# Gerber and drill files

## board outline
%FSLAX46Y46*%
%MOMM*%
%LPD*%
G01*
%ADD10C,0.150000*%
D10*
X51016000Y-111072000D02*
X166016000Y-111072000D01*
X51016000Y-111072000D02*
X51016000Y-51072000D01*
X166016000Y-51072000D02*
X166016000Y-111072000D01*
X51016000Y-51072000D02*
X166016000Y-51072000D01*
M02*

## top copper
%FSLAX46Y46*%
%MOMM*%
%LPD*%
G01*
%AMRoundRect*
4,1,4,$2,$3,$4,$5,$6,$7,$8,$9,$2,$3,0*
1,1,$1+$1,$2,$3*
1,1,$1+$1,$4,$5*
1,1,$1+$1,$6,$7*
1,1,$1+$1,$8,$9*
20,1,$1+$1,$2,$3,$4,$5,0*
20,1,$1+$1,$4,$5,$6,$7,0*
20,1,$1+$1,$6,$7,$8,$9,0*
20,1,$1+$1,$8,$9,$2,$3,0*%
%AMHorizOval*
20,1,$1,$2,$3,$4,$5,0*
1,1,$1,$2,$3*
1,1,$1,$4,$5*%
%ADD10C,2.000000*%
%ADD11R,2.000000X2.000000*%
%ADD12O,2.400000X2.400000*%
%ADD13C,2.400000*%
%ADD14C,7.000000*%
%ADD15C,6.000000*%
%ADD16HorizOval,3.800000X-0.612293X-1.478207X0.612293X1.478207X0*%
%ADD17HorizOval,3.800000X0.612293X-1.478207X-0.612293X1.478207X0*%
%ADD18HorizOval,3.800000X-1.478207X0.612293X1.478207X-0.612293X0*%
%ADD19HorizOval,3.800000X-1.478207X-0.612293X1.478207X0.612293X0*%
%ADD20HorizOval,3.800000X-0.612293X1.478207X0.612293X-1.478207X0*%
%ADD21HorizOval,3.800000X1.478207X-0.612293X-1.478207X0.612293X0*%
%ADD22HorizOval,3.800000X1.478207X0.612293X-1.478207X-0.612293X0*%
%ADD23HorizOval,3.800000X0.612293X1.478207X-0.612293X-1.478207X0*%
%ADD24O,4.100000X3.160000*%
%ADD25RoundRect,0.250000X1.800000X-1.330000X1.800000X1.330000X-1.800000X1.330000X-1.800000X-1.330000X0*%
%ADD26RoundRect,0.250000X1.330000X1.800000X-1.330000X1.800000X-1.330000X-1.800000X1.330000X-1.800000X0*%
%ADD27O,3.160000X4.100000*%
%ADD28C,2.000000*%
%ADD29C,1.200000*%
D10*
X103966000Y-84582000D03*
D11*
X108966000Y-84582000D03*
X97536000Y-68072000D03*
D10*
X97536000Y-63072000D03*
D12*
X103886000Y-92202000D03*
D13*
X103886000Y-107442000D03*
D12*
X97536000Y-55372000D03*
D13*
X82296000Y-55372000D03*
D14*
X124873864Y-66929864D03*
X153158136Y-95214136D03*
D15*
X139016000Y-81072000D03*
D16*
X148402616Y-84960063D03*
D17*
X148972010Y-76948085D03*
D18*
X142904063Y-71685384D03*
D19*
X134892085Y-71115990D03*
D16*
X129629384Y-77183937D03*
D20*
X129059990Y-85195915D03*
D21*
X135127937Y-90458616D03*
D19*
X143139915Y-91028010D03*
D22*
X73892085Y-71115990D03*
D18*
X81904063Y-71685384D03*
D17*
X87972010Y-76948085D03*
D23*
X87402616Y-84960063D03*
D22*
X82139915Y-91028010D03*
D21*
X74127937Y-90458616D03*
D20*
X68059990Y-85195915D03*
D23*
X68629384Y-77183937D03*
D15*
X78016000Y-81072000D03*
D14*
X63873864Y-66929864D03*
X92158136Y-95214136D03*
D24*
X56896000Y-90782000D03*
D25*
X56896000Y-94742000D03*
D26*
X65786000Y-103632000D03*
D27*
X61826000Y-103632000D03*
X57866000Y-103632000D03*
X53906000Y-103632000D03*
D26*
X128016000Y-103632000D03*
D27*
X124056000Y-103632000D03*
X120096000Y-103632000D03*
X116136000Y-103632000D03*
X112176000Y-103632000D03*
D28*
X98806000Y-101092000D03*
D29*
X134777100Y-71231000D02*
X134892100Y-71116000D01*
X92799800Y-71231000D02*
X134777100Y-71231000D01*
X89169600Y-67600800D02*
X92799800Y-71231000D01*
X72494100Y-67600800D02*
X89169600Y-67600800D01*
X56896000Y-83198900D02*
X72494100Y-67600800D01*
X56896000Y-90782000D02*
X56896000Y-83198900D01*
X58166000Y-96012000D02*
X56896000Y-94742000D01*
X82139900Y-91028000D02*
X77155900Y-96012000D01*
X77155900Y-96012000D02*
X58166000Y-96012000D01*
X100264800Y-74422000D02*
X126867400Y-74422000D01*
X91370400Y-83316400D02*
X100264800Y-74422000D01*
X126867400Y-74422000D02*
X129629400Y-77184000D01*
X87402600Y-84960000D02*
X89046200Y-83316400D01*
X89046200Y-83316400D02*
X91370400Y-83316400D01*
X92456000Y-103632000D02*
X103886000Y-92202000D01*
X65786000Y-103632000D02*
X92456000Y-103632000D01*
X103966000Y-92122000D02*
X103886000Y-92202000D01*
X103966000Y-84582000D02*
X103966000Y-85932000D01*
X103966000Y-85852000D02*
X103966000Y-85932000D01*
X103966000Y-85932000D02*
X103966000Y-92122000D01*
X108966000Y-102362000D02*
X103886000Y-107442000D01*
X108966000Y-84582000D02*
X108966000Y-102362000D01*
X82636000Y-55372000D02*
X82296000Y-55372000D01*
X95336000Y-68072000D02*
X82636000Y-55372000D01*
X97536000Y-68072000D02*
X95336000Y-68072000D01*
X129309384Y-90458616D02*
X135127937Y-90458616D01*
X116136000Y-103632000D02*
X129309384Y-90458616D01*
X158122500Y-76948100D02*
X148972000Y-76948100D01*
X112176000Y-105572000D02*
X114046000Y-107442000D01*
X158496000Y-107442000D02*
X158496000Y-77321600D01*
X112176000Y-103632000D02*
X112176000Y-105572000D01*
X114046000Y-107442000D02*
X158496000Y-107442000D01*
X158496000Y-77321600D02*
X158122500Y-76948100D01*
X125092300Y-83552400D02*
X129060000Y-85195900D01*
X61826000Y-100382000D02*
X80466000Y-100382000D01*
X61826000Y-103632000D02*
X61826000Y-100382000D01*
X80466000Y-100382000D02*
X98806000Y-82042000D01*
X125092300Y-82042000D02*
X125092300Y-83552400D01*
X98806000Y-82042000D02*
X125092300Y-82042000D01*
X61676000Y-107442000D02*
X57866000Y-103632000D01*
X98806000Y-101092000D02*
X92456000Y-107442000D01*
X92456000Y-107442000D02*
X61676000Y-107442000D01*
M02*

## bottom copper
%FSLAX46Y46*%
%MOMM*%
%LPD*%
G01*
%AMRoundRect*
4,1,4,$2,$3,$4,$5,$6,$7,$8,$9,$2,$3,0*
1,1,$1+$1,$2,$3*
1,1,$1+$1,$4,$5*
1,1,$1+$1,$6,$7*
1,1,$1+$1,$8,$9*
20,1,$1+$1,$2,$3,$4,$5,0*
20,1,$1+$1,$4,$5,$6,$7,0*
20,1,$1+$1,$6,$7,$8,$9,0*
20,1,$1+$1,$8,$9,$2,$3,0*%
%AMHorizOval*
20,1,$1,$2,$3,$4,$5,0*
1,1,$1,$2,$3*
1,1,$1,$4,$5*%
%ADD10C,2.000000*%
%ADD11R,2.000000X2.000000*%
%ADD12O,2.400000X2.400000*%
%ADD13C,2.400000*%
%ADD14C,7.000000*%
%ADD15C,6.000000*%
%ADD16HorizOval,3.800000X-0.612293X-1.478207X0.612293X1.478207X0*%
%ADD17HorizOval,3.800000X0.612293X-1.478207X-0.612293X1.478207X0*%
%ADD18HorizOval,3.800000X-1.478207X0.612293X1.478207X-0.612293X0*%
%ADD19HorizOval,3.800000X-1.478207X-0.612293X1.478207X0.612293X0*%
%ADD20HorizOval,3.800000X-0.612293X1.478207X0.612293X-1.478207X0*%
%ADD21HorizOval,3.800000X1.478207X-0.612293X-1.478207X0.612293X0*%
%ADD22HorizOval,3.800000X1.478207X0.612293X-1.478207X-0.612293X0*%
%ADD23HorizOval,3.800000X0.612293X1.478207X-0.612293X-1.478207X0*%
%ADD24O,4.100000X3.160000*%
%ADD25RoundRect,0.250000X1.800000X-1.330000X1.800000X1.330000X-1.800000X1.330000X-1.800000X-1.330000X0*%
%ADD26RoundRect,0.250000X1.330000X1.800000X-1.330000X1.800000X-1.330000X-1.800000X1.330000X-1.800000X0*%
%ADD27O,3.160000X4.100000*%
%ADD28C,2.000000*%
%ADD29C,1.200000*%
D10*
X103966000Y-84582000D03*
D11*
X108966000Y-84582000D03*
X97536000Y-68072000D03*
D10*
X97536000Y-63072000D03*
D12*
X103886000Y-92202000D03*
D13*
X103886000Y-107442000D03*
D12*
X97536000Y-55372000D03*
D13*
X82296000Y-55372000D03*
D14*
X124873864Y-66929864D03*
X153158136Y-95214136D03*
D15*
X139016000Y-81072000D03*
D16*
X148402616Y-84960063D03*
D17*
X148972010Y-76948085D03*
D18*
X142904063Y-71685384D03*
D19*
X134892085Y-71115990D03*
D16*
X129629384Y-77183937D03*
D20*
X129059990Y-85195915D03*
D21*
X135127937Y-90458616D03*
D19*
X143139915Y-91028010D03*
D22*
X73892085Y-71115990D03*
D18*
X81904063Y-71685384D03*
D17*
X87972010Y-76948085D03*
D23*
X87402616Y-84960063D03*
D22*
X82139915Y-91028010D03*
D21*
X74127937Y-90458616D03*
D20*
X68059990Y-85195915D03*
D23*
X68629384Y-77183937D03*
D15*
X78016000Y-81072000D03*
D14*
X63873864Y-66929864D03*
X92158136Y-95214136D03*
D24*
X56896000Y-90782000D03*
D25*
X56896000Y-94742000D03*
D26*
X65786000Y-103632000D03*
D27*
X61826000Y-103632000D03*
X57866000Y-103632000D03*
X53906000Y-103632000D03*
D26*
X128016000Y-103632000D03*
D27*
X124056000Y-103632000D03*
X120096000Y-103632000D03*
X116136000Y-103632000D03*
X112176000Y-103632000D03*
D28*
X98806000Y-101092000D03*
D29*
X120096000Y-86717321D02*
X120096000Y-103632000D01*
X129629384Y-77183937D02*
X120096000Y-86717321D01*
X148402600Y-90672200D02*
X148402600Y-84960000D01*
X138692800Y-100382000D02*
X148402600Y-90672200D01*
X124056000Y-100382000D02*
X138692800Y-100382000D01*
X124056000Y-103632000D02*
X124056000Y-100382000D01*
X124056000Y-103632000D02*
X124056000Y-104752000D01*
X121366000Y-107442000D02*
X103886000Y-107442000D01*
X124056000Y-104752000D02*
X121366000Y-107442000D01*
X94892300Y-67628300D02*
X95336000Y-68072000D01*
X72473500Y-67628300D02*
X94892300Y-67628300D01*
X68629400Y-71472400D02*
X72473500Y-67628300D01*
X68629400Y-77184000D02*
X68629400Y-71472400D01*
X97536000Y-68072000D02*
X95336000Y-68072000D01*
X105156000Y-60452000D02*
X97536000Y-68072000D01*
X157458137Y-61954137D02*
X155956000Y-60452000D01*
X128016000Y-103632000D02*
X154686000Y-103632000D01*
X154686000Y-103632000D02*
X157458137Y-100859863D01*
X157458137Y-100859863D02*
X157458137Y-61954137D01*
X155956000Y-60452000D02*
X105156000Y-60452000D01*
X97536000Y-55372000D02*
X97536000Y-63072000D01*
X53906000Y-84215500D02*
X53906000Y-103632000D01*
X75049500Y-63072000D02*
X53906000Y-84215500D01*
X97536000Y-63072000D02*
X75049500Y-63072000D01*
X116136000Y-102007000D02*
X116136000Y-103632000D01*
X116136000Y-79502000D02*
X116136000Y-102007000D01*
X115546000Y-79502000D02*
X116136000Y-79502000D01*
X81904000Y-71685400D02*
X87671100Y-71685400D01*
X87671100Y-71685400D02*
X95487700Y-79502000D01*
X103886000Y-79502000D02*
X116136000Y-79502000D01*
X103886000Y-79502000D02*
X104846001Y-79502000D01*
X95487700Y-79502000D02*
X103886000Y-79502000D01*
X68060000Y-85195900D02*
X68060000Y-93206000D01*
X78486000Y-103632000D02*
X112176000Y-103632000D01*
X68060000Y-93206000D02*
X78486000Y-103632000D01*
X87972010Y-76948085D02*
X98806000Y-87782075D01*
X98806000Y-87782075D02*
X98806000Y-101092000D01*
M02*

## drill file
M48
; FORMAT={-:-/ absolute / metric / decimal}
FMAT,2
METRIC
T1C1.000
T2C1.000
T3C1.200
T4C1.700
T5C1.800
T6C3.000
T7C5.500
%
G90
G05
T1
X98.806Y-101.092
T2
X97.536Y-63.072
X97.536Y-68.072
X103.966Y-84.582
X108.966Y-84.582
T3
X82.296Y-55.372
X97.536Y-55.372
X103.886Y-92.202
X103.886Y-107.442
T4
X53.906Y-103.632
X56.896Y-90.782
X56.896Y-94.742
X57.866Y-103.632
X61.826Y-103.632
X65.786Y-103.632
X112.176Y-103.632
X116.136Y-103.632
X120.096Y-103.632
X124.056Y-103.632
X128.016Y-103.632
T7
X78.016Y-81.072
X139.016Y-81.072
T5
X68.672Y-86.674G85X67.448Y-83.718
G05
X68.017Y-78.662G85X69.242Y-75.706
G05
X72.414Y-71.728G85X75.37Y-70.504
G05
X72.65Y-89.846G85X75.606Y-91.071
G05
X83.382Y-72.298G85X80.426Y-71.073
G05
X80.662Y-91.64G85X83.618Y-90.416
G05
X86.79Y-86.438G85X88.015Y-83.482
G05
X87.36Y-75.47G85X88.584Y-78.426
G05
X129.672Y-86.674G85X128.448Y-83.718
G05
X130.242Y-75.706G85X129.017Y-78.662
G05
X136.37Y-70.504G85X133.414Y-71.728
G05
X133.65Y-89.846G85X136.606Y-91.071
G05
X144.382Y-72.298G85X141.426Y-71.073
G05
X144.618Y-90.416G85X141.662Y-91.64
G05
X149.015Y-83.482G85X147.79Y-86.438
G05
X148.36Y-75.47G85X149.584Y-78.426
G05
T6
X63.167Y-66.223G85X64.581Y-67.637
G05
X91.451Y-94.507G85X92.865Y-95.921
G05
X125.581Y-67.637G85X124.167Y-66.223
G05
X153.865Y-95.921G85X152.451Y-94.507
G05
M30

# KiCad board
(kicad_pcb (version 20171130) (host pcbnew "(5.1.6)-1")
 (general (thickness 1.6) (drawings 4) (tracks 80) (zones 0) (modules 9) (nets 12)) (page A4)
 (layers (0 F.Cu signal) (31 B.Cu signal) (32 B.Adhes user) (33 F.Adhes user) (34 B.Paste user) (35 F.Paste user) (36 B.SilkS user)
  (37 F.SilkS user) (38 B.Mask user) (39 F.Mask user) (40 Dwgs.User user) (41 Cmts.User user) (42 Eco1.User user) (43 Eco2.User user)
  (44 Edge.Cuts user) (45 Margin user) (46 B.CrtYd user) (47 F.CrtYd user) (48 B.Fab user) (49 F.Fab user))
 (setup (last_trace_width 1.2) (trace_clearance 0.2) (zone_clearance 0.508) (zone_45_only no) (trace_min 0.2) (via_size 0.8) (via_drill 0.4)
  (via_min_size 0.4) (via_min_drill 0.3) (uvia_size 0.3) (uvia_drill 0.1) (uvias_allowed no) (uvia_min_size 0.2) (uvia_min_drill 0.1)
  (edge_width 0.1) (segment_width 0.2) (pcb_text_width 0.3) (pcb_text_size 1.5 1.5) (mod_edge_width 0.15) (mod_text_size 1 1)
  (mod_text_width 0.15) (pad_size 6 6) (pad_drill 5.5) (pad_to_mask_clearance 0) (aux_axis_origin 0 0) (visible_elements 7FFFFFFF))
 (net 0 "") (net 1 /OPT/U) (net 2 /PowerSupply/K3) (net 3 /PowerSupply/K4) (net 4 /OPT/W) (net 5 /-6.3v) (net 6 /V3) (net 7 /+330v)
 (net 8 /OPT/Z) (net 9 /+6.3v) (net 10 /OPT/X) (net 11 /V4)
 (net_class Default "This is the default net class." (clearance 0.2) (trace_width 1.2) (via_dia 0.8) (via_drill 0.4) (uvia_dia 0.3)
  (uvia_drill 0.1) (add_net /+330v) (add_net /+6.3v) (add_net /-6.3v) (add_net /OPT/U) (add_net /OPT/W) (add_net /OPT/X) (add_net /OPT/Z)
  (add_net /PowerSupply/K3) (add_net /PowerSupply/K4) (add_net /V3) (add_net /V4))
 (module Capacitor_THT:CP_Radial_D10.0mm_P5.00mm (layer F.Cu) (at 108.966 84.582 180)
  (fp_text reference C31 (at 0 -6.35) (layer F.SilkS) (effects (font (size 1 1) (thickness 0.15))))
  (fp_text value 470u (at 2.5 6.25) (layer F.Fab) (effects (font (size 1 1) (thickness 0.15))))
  (pad 2 thru_hole circle (at 5 0 180) (size 2 2) (drill 1) (layers *.Cu *.Mask) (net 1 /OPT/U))
  (pad 1 thru_hole rect (at 0 0 180) (size 2 2) (drill 1) (layers *.Cu *.Mask) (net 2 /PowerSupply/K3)))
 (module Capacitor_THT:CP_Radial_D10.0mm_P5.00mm (layer F.Cu) (at 97.536 68.072 90)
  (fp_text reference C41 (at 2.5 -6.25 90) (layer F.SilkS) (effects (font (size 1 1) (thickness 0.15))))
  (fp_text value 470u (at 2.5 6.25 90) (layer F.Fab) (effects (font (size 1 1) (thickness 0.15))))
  (pad 1 thru_hole rect (at 0 0 90) (size 2 2) (drill 1) (layers *.Cu *.Mask) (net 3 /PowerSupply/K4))
  (pad 2 thru_hole circle (at 5 0 90) (size 2 2) (drill 1) (layers *.Cu *.Mask) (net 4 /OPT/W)))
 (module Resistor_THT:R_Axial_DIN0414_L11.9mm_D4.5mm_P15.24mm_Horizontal (layer F.Cu) (at 103.886 107.442 90)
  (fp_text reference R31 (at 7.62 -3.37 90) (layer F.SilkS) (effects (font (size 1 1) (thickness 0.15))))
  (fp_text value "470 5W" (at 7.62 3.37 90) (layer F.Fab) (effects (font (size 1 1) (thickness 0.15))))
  (pad 2 thru_hole oval (at 15.24 0 90) (size 2.4 2.4) (drill 1.2) (layers *.Cu *.Mask) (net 1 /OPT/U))
  (pad 1 thru_hole circle (at 0 0 90) (size 2.4 2.4) (drill 1.2) (layers *.Cu *.Mask) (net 2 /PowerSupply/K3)))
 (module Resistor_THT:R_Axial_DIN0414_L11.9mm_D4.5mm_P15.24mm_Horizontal (layer F.Cu) (at 82.296 55.372)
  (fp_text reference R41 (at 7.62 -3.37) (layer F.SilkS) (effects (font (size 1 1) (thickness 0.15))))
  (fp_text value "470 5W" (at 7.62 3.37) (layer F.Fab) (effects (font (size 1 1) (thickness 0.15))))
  (pad 2 thru_hole oval (at 15.24 0) (size 2.4 2.4) (drill 1.2) (layers *.Cu *.Mask) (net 4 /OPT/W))
  (pad 1 thru_hole circle (at 0 0) (size 2.4 2.4) (drill 1.2) (layers *.Cu *.Mask) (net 3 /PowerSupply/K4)))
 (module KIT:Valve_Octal (layer B.Cu) (at 139.016 81.072 135)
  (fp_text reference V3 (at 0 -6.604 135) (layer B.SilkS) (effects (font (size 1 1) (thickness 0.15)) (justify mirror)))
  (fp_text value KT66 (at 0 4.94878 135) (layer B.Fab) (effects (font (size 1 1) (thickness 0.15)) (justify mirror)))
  (pad 10 thru_hole circle (at 20 0 135) (size 7 7) (drill oval 5 3) (layers *.Cu *.Mask))
  (pad 9 thru_hole circle (at -20 0 135) (size 7 7) (drill oval 5 3) (layers *.Cu *.Mask))
  (pad "" thru_hole circle (at 0 0 247.5) (size 6 6) (drill 5.5) (layers *.Cu *.Mask))
  (pad 8 thru_hole oval (at -9.386616 3.888064 247.5) (size 7 3.8) (drill oval 5 1.8) (layers *.Cu *.Mask) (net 2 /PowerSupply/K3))
  (pad 7 thru_hole oval (at -4.123914 9.95601 292.5) (size 7 3.8) (drill oval 5 1.8) (layers *.Cu *.Mask) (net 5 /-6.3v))
  (pad 6 thru_hole oval (at 3.888064 9.386616 157.5) (size 7 3.8) (drill oval 5 1.8) (layers *.Cu *.Mask))
  (pad 5 thru_hole oval (at 9.95601 4.123914 202.5) (size 7 3.8) (drill oval 5 1.8) (layers *.Cu *.Mask) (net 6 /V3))
  (pad 4 thru_hole oval (at 9.386616 -3.888064 247.5) (size 7 3.8) (drill oval 5 1.8) (layers *.Cu *.Mask) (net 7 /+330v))
  (pad 3 thru_hole oval (at 4.123914 -9.95601 112.5) (size 7 3.8) (drill oval 5 1.8) (layers *.Cu *.Mask) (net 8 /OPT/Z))
  (pad 2 thru_hole oval (at -3.888064 -9.386616 337.5) (size 7 3.8) (drill oval 5 1.8) (layers *.Cu *.Mask) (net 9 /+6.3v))
  (pad 1 thru_hole oval (at -9.95601 -4.123914 202.5) (size 7 3.8) (drill oval 5 1.8) (layers *.Cu *.Mask)))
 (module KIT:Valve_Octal (layer B.Cu) (at 78.016 81.072 315)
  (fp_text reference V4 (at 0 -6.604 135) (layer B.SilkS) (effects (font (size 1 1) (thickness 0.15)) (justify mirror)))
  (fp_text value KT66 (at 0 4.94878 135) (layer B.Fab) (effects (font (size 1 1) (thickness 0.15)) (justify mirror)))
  (pad 1 thru_hole oval (at -9.95601 -4.123914 22.5) (size 7 3.8) (drill oval 5 1.8) (layers *.Cu *.Mask))
  (pad 2 thru_hole oval (at -3.888064 -9.386616 157.5) (size 7 3.8) (drill oval 5 1.8) (layers *.Cu *.Mask) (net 9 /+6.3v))
  (pad 3 thru_hole oval (at 4.123914 -9.95601 292.5) (size 7 3.8) (drill oval 5 1.8) (layers *.Cu *.Mask) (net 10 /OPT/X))
  (pad 4 thru_hole oval (at 9.386616 -3.888064 67.5) (size 7 3.8) (drill oval 5 1.8) (layers *.Cu *.Mask) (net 7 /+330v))
  (pad 5 thru_hole oval (at 9.95601 4.123914 22.5) (size 7 3.8) (drill oval 5 1.8) (layers *.Cu *.Mask) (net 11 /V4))
  (pad 6 thru_hole oval (at 3.888064 9.386616 337.5) (size 7 3.8) (drill oval 5 1.8) (layers *.Cu *.Mask))
  (pad 7 thru_hole oval (at -4.123914 9.95601 112.5) (size 7 3.8) (drill oval 5 1.8) (layers *.Cu *.Mask) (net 5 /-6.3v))
  (pad 8 thru_hole oval (at -9.386616 3.888064 67.5) (size 7 3.8) (drill oval 5 1.8) (layers *.Cu *.Mask) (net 3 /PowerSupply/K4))
  (pad "" thru_hole circle (at 0 0 67.5) (size 6 6) (drill 5.5) (layers *.Cu *.Mask))
  (pad 9 thru_hole circle (at -20 0 315) (size 7 7) (drill oval 5 3) (layers *.Cu *.Mask))
  (pad 10 thru_hole circle (at 20 0 315) (size 7 7) (drill oval 5 3) (layers *.Cu *.Mask)))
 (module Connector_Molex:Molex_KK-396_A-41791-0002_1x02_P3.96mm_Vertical (layer F.Cu) (at 56.896 94.742 90)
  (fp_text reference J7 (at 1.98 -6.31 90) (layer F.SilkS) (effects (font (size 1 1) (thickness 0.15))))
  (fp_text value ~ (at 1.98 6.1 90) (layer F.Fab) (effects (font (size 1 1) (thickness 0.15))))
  (pad 2 thru_hole oval (at 3.96 0 90) (size 3.16 4.1) (drill 1.7) (layers *.Cu *.Mask) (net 6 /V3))
  (pad 1 thru_hole roundrect (at 0 0 90) (size 3.16 4.1) (drill 1.7) (layers *.Cu *.Mask) (roundrect_rratio 0.079114) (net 11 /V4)))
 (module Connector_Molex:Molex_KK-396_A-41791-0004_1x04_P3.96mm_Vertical (layer F.Cu) (at 65.786 103.632 180)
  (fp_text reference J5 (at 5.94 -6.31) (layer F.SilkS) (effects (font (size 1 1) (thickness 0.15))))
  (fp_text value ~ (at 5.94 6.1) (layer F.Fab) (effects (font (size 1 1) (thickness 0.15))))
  (pad 1 thru_hole roundrect (at 0 0 180) (size 3.16 4.1) (drill 1.7) (layers *.Cu *.Mask) (roundrect_rratio 0.079114) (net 1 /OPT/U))
  (pad 2 thru_hole oval (at 3.96 0 180) (size 3.16 4.1) (drill 1.7) (layers *.Cu *.Mask) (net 8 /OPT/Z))
  (pad 3 thru_hole oval (at 7.92 0 180) (size 3.16 4.1) (drill 1.7) (layers *.Cu *.Mask) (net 10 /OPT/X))
  (pad 4 thru_hole oval (at 11.88 0 180) (size 3.16 4.1) (drill 1.7) (layers *.Cu *.Mask) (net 4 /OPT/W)))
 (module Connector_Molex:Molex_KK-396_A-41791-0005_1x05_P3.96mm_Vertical (layer F.Cu) (at 128.016 103.632 180)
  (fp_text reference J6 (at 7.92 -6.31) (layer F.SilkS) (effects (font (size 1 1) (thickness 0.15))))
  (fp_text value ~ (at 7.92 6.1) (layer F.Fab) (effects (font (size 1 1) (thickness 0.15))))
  (pad 1 thru_hole roundrect (at 0 0 180) (size 3.16 4.1) (drill 1.7) (layers *.Cu *.Mask) (roundrect_rratio 0.079114)
   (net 3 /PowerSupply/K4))
  (pad 2 thru_hole oval (at 3.96 0 180) (size 3.16 4.1) (drill 1.7) (layers *.Cu *.Mask) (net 2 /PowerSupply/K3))
  (pad 3 thru_hole oval (at 7.92 0 180) (size 3.16 4.1) (drill 1.7) (layers *.Cu *.Mask) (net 7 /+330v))
  (pad 4 thru_hole oval (at 11.88 0 180) (size 3.16 4.1) (drill 1.7) (layers *.Cu *.Mask) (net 9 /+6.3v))
  (pad 5 thru_hole oval (at 15.84 0 180) (size 3.16 4.1) (drill 1.7) (layers *.Cu *.Mask) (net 5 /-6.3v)))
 (gr_line (start 51.016 111.072) (end 166.016 111.072) (layer Edge.Cuts) (width 0.15))
 (gr_line (start 51.016 111.072) (end 51.016 51.072) (layer Edge.Cuts) (width 0.15))
 (gr_line (start 166.016 51.072) (end 166.016 111.072) (layer Edge.Cuts) (width 0.15))
 (gr_line (start 51.016 51.072) (end 166.016 51.072) (layer Edge.Cuts) (width 0.15))
 (segment (start 134.7771 71.231) (end 134.8921 71.116) (width 1.2) (layer F.Cu) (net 6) (status 30))
 (segment (start 92.7998 71.231) (end 134.7771 71.231) (width 1.2) (layer F.Cu) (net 6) (status 20))
 (segment (start 89.1696 67.6008) (end 92.7998 71.231) (width 1.2) (layer F.Cu) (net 6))
 (segment (start 72.4941 67.6008) (end 89.1696 67.6008) (width 1.2) (layer F.Cu) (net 6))
 (segment (start 56.896 83.1989) (end 72.4941 67.6008) (width 1.2) (layer F.Cu) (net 6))
 (segment (start 56.896 90.782) (end 56.896 83.1989) (width 1.2) (layer F.Cu) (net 6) (status 10))
 (segment (start 58.166 96.012) (end 56.896 94.742) (width 1.2) (layer F.Cu) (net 11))
 (segment (start 82.1399 91.028) (end 77.1559 96.012) (width 1.2) (layer F.Cu) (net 11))
 (segment (start 77.1559 96.012) (end 58.166 96.012) (width 1.2) (layer F.Cu) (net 11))
 (segment (start 120.096 86.717321) (end 120.096 103.632) (width 1.2) (layer B.Cu) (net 7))
 (segment (start 129.629384 77.183937) (end 120.096 86.717321) (width 1.2) (layer B.Cu) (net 7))
 (segment (start 100.2648 74.422) (end 126.8674 74.422) (width 1.2) (layer F.Cu) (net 7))
 (segment (start 91.3704 83.3164) (end 100.2648 74.422) (width 1.2) (layer F.Cu) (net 7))
 (segment (start 126.8674 74.422) (end 129.6294 77.184) (width 1.2) (layer F.Cu) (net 7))
 (segment (start 87.4026 84.96) (end 89.0462 83.3164) (width 1.2) (layer F.Cu) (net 7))
 (segment (start 89.0462 83.3164) (end 91.3704 83.3164) (width 1.2) (layer F.Cu) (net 7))
 (segment (start 92.456 103.632) (end 103.886 92.202) (width 1.2) (layer F.Cu) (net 1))
 (segment (start 65.786 103.632) (end 92.456 103.632) (width 1.2) (layer F.Cu) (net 1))
 (segment (start 103.966 92.122) (end 103.886 92.202) (width 1.2) (layer F.Cu) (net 1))
 (segment (start 103.966 84.582) (end 103.966 85.932) (width 1.2) (layer F.Cu) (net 1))
 (segment (start 103.966 85.852) (end 103.966 85.932) (width 1.2) (layer F.Cu) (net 1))
 (segment (start 103.966 85.932) (end 103.966 92.122) (width 1.2) (layer F.Cu) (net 1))
 (segment (start 148.4026 90.6722) (end 148.4026 84.96) (width 1.2) (layer B.Cu) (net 2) (status 20))
 (segment (start 138.6928 100.382) (end 148.4026 90.6722) (width 1.2) (layer B.Cu) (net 2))
 (segment (start 124.056 100.382) (end 138.6928 100.382) (width 1.2) (layer B.Cu) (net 2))
 (segment (start 124.056 103.632) (end 124.056 100.382) (width 1.2) (layer B.Cu) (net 2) (status 10))
 (segment (start 124.056 103.632) (end 124.056 104.752) (width 1.2) (layer B.Cu) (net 2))
 (segment (start 121.366 107.442) (end 103.886 107.442) (width 1.2) (layer B.Cu) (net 2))
 (segment (start 124.056 104.752) (end 121.366 107.442) (width 1.2) (layer B.Cu) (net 2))
 (segment (start 108.966 102.362) (end 103.886 107.442) (width 1.2) (layer F.Cu) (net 2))
 (segment (start 108.966 84.582) (end 108.966 102.362) (width 1.2) (layer F.Cu) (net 2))
 (segment (start 94.8923 67.6283) (end 95.336 68.072) (width 1.2) (layer B.Cu) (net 3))
 (segment (start 72.4735 67.6283) (end 94.8923 67.6283) (width 1.2) (layer B.Cu) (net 3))
 (segment (start 68.6294 71.4724) (end 72.4735 67.6283) (width 1.2) (layer B.Cu) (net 3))
 (segment (start 68.6294 77.184) (end 68.6294 71.4724) (width 1.2) (layer B.Cu) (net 3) (status 10))
 (segment (start 97.536 68.072) (end 95.336 68.072) (width 1.2) (layer B.Cu) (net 3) (status 10))
 (segment (start 82.636 55.372) (end 82.296 55.372) (width 1.2) (layer F.Cu) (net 3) (status 30))
 (segment (start 95.336 68.072) (end 82.636 55.372) (width 1.2) (layer F.Cu) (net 3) (status 20))
 (segment (start 97.536 68.072) (end 95.336 68.072) (width 1.2) (layer F.Cu) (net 3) (status 10))
 (segment (start 105.156 60.452) (end 97.536 68.072) (width 1.2) (layer B.Cu) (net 3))
 (segment (start 157.458137 61.954137) (end 155.956 60.452) (width 1.2) (layer B.Cu) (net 3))
 (segment (start 128.016 103.632) (end 154.686 103.632) (width 1.2) (layer B.Cu) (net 3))
 (segment (start 154.686 103.632) (end 157.458137 100.859863) (width 1.2) (layer B.Cu) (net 3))
 (segment (start 157.458137 100.859863) (end 157.458137 61.954137) (width 1.2) (layer B.Cu) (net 3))
 (segment (start 155.956 60.452) (end 105.156 60.452) (width 1.2) (layer B.Cu) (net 3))
 (segment (start 97.536 55.372) (end 97.536 63.072) (width 1.2) (layer B.Cu) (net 4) (status 30))
 (segment (start 53.906 84.2155) (end 53.906 103.632) (width 1.2) (layer B.Cu) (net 4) (status 20))
 (segment (start 75.0495 63.072) (end 53.906 84.2155) (width 1.2) (layer B.Cu) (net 4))
 (segment (start 97.536 63.072) (end 75.0495 63.072) (width 1.2) (layer B.Cu) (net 4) (status 10))
 (segment (start 129.309384 90.458616) (end 135.127937 90.458616) (width 1.2) (layer F.Cu) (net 9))
 (segment (start 116.136 103.632) (end 129.309384 90.458616) (width 1.2) (layer F.Cu) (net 9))
 (segment (start 116.136 102.007) (end 116.136 103.632) (width 1.2) (layer B.Cu) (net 9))
 (segment (start 116.136 79.502) (end 116.136 102.007) (width 1.2) (layer B.Cu) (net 9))
 (segment (start 115.546 79.502) (end 116.136 79.502) (width 1.2) (layer B.Cu) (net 9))
 (segment (start 81.904 71.6854) (end 87.6711 71.6854) (width 1.2) (layer B.Cu) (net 9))
 (segment (start 87.6711 71.6854) (end 95.4877 79.502) (width 1.2) (layer B.Cu) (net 9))
 (segment (start 103.886 79.502) (end 116.136 79.502) (width 1.2) (layer B.Cu) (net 9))
 (segment (start 103.886 79.502) (end 104.846001 79.502) (width 1.2) (layer B.Cu) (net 9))
 (segment (start 95.4877 79.502) (end 103.886 79.502) (width 1.2) (layer B.Cu) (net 9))
 (segment (start 68.06 85.1959) (end 68.06 93.206) (width 1.2) (layer B.Cu) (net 5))
 (segment (start 78.486 103.632) (end 112.176 103.632) (width 1.2) (layer B.Cu) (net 5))
 (segment (start 68.06 93.206) (end 78.486 103.632) (width 1.2) (layer B.Cu) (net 5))
 (segment (start 158.1225 76.9481) (end 148.972 76.9481) (width 1.2) (layer F.Cu) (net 5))
 (segment (start 112.176 105.572) (end 114.046 107.442) (width 1.2) (layer F.Cu) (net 5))
 (segment (start 158.496 107.442) (end 158.496 77.3216) (width 1.2) (layer F.Cu) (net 5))
 (segment (start 112.176 103.632) (end 112.176 105.572) (width 1.2) (layer F.Cu) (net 5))
 (segment (start 114.046 107.442) (end 158.496 107.442) (width 1.2) (layer F.Cu) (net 5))
 (segment (start 158.496 77.3216) (end 158.1225 76.9481) (width 1.2) (layer F.Cu) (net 5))
 (segment (start 125.0923 83.5524) (end 129.06 85.1959) (width 1.2) (layer F.Cu) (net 8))
 (segment (start 61.826 100.382) (end 80.466 100.382) (width 1.2) (layer F.Cu) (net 8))
 (segment (start 61.826 103.632) (end 61.826 100.382) (width 1.2) (layer F.Cu) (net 8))
 (segment (start 80.466 100.382) (end 98.806 82.042) (width 1.2) (layer F.Cu) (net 8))
 (segment (start 125.0923 82.042) (end 125.0923 83.5524) (width 1.2) (layer F.Cu) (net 8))
 (segment (start 98.806 82.042) (end 125.0923 82.042) (width 1.2) (layer F.Cu) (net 8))
 (via (at 98.806 101.092) (size 2) (drill 1) (layers F.Cu B.Cu) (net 10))
 (segment (start 87.97201 76.948085) (end 98.806 87.782075) (width 1.2) (layer B.Cu) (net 10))
 (segment (start 98.806 87.782075) (end 98.806 101.092) (width 1.2) (layer B.Cu) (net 10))
 (segment (start 61.676 107.442) (end 57.866 103.632) (width 1.2) (layer F.Cu) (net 10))
 (segment (start 98.806 101.092) (end 92.456 107.442) (width 1.2) (layer F.Cu) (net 10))
 (segment (start 92.456 107.442) (end 61.676 107.442) (width 1.2) (layer F.Cu) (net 10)))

